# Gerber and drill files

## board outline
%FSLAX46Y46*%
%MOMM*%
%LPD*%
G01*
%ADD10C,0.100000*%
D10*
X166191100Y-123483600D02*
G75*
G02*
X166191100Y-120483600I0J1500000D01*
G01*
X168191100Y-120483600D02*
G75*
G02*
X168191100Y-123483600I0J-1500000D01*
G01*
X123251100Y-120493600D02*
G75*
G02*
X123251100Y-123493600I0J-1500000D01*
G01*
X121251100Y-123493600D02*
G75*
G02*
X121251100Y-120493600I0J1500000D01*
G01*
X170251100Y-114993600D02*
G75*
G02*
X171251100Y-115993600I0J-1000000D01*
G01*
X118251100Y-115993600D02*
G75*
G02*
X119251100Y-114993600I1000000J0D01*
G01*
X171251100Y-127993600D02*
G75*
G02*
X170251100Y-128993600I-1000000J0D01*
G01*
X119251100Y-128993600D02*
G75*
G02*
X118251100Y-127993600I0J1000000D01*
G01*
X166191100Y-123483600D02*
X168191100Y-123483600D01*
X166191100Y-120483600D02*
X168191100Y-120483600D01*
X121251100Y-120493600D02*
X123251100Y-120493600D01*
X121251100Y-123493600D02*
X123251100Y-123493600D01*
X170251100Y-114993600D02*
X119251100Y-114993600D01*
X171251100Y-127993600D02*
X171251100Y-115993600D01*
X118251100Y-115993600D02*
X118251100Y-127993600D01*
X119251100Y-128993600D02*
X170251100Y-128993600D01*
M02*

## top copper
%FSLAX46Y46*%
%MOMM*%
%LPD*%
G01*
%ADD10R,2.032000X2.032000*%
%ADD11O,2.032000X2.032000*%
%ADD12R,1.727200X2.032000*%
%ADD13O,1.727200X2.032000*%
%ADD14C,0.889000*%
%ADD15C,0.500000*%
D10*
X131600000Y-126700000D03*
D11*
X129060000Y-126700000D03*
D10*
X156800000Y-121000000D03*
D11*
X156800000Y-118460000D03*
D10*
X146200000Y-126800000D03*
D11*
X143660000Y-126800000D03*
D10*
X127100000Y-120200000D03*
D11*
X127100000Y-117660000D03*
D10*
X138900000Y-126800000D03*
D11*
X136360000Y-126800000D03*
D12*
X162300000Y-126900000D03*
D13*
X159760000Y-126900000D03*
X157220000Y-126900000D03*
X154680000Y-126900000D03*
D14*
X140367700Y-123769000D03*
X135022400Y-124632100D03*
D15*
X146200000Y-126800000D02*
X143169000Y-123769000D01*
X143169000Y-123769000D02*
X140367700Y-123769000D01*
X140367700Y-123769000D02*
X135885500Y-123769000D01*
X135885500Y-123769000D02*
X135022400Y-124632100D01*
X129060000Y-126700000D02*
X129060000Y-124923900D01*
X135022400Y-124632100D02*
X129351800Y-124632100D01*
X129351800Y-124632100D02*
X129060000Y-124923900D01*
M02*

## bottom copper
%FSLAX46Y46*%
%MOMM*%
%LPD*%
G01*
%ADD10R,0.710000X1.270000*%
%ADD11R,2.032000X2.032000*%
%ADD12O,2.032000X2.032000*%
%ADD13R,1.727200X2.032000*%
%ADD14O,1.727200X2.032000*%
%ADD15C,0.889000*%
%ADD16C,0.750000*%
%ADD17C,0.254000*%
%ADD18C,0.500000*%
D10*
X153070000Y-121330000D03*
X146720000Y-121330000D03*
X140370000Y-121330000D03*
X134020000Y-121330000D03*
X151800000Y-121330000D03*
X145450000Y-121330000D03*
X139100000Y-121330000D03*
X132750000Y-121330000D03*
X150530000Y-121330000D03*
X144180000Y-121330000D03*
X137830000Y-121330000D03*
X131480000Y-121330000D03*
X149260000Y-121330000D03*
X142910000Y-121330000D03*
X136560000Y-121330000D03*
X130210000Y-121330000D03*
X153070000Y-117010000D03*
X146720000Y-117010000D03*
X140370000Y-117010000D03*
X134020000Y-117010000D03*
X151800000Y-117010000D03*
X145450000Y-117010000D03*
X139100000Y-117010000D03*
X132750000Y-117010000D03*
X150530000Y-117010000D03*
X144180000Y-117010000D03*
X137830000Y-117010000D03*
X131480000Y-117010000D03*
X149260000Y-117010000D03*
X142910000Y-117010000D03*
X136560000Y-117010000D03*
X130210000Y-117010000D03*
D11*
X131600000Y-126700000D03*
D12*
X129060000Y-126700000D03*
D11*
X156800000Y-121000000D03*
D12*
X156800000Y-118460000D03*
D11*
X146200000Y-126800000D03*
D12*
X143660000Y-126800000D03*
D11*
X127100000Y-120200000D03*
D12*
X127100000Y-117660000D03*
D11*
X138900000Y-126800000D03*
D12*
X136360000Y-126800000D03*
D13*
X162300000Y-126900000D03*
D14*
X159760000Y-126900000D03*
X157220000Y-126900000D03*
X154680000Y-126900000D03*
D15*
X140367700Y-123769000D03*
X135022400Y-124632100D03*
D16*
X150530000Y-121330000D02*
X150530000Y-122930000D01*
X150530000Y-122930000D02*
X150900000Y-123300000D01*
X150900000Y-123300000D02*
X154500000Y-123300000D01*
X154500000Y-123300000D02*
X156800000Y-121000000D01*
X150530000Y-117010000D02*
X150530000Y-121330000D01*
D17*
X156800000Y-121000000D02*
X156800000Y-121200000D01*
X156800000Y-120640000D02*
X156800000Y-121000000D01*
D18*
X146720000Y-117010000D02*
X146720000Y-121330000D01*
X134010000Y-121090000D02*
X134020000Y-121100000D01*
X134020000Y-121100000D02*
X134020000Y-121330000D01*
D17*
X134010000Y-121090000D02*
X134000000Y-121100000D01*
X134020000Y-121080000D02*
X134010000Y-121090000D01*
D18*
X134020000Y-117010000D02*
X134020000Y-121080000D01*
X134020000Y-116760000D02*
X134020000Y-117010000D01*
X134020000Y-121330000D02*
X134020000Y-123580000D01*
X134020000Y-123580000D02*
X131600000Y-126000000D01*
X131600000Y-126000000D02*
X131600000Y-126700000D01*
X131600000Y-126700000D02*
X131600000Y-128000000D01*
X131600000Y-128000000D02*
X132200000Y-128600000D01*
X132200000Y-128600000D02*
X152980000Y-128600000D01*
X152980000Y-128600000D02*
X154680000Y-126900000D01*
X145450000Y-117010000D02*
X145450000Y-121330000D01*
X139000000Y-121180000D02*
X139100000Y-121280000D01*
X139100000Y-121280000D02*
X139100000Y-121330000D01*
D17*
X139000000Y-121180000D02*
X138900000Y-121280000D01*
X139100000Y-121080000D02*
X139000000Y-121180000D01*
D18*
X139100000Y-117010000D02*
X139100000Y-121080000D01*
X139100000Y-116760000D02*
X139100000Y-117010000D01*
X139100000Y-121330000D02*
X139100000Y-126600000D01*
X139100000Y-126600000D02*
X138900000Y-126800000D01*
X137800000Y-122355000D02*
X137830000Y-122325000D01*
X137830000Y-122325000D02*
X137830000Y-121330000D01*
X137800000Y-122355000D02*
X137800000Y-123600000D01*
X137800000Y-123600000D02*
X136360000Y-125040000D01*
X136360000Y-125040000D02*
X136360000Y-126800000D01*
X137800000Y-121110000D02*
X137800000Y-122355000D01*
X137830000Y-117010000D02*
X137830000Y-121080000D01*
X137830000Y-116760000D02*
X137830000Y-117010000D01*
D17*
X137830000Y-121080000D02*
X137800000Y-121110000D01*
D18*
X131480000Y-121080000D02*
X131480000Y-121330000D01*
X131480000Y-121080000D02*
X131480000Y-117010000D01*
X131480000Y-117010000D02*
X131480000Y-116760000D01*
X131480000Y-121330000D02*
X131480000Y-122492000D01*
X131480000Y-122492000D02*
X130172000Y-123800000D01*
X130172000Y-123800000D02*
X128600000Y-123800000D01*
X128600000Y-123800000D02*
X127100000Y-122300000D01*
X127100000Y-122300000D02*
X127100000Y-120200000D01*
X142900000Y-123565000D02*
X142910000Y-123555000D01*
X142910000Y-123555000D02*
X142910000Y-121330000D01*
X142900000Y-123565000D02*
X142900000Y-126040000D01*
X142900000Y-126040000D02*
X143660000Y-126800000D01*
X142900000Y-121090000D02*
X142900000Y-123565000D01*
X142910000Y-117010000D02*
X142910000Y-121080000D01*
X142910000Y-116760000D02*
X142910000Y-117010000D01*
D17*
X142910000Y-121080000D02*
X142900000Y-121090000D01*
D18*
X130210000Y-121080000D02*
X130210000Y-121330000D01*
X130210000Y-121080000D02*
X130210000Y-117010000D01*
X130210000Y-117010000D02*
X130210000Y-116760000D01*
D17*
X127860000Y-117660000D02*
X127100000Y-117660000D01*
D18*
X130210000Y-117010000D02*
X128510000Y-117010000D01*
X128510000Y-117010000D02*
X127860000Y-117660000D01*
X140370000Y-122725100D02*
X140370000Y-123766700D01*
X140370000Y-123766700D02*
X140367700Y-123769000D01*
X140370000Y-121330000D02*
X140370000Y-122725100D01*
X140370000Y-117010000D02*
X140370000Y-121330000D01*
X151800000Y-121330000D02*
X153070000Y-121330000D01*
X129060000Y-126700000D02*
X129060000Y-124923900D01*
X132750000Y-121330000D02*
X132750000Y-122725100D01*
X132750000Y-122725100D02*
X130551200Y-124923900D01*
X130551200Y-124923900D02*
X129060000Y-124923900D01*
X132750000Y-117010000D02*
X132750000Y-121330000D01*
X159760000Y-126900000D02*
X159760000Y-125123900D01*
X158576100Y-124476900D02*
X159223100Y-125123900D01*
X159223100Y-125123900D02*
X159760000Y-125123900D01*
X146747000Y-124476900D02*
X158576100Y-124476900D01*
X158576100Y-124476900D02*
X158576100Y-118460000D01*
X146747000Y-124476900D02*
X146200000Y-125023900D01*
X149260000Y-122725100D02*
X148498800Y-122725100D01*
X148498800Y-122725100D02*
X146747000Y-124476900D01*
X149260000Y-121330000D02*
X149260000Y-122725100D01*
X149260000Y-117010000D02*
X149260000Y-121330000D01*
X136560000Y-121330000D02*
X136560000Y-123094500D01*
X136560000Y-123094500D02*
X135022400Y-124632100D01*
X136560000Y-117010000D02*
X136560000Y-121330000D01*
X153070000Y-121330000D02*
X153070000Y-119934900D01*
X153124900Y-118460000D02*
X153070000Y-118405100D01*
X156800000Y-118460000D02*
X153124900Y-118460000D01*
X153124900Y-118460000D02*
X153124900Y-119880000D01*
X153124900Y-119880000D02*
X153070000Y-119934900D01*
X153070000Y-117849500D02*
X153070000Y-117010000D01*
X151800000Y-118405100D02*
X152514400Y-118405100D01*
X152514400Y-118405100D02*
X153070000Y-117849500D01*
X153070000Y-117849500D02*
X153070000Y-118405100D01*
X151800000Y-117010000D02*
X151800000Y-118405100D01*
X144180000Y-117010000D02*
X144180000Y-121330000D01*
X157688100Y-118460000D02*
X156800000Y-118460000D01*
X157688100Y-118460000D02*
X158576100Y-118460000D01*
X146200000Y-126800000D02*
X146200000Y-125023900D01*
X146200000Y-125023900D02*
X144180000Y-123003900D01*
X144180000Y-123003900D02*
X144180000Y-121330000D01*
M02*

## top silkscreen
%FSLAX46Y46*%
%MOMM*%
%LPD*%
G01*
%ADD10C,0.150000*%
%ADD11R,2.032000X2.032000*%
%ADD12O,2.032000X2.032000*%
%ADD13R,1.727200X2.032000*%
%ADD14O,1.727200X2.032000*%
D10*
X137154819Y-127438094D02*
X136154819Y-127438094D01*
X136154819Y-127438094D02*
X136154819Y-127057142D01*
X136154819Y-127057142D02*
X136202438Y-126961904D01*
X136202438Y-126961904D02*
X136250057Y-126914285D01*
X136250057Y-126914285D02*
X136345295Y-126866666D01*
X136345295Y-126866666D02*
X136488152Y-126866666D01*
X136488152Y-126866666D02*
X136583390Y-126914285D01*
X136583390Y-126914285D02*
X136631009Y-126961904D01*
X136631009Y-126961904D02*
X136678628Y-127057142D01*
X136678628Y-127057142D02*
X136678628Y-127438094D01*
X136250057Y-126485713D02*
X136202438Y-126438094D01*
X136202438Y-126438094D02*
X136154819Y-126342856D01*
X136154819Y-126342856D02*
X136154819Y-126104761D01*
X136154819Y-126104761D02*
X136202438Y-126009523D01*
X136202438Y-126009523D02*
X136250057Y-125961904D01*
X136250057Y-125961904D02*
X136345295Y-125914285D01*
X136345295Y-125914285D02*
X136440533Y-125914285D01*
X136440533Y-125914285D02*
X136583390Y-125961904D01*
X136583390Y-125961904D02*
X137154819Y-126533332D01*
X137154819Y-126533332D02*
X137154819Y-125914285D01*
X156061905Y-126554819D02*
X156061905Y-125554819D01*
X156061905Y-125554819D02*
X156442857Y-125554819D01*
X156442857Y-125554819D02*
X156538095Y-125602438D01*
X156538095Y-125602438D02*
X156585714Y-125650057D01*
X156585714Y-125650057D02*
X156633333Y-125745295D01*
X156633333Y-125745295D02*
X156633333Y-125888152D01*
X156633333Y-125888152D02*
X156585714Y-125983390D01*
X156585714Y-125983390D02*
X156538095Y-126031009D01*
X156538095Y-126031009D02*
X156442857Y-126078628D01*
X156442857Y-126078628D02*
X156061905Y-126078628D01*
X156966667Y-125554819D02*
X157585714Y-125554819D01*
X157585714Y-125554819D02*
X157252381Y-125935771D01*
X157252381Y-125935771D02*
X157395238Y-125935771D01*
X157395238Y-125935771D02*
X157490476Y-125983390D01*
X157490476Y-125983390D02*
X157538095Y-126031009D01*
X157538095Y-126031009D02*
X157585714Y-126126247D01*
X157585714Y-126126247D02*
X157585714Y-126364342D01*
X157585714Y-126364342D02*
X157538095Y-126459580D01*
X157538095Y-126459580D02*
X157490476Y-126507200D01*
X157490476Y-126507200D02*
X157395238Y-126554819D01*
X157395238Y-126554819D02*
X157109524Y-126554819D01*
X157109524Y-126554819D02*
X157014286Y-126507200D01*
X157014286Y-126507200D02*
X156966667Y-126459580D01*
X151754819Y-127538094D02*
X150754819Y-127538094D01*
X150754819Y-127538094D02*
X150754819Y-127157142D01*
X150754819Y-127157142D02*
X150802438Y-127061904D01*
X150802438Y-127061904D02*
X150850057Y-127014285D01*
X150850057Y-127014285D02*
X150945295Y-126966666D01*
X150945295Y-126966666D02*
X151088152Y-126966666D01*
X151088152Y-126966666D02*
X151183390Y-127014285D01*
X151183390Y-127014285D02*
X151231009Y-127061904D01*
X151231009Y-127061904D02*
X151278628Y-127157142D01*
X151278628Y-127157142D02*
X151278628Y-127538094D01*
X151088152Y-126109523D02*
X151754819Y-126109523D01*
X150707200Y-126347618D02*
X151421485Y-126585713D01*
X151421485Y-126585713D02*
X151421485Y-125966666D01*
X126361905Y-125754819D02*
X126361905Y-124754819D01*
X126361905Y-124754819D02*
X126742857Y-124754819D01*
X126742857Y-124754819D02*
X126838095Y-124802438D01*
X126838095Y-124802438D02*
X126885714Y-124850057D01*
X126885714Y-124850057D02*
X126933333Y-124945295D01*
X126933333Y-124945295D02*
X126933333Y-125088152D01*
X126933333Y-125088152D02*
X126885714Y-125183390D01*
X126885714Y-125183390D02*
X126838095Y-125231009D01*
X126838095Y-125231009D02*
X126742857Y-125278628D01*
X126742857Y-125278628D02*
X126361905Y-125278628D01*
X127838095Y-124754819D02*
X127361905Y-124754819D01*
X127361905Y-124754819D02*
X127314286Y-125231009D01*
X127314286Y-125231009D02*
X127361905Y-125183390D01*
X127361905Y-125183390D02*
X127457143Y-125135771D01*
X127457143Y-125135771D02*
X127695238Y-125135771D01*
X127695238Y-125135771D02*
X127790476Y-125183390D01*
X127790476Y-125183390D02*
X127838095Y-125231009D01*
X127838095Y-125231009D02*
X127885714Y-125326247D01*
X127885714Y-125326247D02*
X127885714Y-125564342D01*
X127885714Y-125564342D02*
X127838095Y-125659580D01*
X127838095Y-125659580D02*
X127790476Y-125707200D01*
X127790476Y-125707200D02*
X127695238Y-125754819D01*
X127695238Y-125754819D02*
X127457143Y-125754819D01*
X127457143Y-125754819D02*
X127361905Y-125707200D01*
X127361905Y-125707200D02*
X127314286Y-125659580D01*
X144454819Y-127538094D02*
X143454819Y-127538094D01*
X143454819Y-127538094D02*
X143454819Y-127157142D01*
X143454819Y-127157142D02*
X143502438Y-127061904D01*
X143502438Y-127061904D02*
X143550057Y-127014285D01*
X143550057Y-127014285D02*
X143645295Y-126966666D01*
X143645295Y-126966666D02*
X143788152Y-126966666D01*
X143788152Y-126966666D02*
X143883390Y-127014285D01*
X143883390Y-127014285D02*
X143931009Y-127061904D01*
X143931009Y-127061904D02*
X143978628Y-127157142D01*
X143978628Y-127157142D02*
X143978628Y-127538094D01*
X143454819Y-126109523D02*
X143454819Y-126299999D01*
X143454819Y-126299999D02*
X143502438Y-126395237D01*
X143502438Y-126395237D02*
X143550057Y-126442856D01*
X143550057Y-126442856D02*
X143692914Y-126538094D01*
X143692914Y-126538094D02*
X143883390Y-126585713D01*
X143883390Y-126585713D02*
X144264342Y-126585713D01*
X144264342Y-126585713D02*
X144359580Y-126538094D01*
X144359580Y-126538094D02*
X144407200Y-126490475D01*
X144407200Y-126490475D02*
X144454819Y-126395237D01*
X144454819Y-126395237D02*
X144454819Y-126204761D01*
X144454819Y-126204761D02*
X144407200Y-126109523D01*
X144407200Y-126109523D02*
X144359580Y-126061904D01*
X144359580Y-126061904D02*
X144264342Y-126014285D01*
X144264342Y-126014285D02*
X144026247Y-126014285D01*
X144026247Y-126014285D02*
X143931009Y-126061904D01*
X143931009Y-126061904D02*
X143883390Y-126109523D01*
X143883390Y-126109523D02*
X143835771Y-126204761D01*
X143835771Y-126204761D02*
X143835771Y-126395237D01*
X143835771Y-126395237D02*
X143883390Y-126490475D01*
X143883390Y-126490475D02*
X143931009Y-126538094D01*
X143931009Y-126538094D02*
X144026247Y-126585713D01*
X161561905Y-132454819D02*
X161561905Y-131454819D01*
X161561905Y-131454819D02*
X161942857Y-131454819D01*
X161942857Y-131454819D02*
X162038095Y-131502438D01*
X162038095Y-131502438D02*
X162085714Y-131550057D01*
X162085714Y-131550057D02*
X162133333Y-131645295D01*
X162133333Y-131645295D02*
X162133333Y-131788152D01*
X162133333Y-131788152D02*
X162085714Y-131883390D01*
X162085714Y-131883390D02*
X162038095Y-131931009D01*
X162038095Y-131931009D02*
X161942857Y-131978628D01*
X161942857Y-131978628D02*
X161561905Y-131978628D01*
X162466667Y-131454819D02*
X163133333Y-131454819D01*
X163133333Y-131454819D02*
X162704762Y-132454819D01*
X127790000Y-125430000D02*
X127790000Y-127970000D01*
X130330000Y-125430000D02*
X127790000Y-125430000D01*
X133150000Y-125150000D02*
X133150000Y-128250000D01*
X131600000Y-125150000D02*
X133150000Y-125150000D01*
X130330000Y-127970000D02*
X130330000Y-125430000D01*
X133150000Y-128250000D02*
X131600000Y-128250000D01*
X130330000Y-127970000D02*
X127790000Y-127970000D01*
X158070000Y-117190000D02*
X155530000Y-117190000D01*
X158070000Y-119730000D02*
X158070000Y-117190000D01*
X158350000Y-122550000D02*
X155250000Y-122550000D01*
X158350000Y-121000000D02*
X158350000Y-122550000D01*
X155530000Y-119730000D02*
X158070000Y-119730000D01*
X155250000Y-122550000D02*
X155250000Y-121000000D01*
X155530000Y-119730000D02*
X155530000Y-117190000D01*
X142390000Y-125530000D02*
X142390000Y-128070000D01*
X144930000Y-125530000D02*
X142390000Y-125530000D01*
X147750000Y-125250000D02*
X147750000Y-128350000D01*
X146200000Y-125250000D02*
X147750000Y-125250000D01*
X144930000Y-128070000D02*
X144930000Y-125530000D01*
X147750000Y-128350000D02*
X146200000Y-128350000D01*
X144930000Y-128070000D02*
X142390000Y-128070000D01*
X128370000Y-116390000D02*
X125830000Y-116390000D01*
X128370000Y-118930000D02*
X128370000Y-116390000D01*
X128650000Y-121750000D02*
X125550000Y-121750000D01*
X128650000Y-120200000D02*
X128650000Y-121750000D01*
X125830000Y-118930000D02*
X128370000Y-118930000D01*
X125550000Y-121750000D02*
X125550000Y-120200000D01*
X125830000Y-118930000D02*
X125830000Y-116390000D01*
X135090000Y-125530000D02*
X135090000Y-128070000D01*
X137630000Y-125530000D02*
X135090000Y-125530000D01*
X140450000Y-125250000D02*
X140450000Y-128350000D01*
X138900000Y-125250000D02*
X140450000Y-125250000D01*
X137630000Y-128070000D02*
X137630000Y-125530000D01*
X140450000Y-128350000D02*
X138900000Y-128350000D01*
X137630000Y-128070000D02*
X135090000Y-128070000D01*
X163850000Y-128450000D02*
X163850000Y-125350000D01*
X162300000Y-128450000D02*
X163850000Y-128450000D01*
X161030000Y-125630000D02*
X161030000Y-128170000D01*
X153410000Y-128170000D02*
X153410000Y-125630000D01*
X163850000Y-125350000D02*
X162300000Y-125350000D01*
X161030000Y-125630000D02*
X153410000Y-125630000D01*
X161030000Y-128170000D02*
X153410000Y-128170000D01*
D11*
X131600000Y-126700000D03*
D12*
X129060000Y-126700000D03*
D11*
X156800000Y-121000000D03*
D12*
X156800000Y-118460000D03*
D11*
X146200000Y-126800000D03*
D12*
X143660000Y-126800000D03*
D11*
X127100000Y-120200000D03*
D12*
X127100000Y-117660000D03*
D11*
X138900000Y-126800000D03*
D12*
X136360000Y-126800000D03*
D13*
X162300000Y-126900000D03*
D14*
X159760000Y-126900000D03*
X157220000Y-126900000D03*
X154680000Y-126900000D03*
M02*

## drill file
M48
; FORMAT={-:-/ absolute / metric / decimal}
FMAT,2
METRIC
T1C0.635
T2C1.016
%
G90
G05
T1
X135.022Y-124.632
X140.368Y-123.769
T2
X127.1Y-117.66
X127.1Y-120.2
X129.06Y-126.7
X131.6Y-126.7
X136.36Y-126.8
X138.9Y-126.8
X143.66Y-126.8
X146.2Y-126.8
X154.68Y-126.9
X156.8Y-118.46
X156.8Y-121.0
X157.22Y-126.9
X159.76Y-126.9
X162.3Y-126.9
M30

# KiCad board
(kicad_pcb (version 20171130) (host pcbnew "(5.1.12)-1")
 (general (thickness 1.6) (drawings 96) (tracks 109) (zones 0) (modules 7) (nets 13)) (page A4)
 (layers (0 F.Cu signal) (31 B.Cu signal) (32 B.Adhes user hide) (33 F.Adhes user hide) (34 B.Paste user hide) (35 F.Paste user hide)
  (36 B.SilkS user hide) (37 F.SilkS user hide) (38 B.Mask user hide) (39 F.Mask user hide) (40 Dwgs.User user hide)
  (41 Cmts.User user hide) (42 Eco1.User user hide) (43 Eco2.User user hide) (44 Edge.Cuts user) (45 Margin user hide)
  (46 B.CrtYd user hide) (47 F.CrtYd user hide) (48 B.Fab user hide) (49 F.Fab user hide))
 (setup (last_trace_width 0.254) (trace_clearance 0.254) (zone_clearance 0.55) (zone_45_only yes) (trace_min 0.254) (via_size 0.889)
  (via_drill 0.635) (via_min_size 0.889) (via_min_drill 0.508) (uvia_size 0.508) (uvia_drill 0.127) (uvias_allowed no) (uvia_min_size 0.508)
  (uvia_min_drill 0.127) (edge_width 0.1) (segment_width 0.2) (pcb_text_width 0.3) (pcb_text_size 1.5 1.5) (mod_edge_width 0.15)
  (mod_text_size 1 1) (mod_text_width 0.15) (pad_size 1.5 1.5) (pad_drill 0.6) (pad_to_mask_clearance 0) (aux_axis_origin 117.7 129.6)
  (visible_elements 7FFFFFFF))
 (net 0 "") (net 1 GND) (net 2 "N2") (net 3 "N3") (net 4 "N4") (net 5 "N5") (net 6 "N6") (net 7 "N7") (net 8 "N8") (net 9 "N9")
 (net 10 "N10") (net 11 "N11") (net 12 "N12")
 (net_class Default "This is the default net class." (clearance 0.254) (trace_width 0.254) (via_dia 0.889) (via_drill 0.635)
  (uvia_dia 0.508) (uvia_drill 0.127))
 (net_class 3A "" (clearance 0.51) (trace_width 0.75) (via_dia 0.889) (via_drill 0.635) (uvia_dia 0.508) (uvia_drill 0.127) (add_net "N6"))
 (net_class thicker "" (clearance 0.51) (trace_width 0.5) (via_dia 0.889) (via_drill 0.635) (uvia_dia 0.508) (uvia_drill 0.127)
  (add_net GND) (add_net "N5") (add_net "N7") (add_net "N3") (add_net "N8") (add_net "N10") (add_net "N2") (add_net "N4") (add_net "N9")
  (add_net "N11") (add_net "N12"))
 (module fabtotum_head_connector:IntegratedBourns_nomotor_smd (layer B.Cu) (at 153 121.35 90)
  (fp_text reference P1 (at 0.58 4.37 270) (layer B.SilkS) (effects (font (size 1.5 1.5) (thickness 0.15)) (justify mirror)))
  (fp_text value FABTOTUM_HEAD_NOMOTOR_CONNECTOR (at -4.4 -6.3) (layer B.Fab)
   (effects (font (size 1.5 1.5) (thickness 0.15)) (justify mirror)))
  (pad 1 smd rect (at 0.02 0.07 90) (size 1.27 0.71) (layers B.Cu B.Paste B.Mask) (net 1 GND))
  (pad 5 smd rect (at 0.02 -6.28 90) (size 1.27 0.71) (layers B.Cu B.Paste B.Mask) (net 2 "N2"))
  (pad 9 smd rect (at 0.02 -12.63 90) (size 1.27 0.71) (layers B.Cu B.Paste B.Mask) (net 1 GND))
  (pad 13 smd rect (at 0.02 -18.98 90) (size 1.27 0.71) (layers B.Cu B.Paste B.Mask) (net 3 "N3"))
  (pad 2 smd rect (at 0.02 -1.2 90) (size 1.27 0.71) (layers B.Cu B.Paste B.Mask) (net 1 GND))
  (pad 6 smd rect (at 0.02 -7.55 90) (size 1.27 0.71) (layers B.Cu B.Paste B.Mask) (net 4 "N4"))
  (pad 10 smd rect (at 0.02 -13.9 90) (size 1.27 0.71) (layers B.Cu B.Paste B.Mask) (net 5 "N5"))
  (pad 14 smd rect (at 0.02 -20.25 90) (size 1.27 0.71) (layers B.Cu B.Paste B.Mask) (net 1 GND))
  (pad 3 smd rect (at 0.02 -2.47 90) (size 1.27 0.71) (layers B.Cu B.Paste B.Mask) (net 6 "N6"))
  (pad 7 smd rect (at 0.02 -8.82 90) (size 1.27 0.71) (layers B.Cu B.Paste B.Mask) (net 1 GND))
  (pad 11 smd rect (at 0.02 -15.17 90) (size 1.27 0.71) (layers B.Cu B.Paste B.Mask) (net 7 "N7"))
  (pad 15 smd rect (at 0.02 -21.52 90) (size 1.27 0.71) (layers B.Cu B.Paste B.Mask) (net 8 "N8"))
  (pad 4 smd rect (at 0.02 -3.74 90) (size 1.27 0.71) (layers B.Cu B.Paste B.Mask) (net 1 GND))
  (pad 8 smd rect (at 0.02 -10.09 90) (size 1.27 0.71) (layers B.Cu B.Paste B.Mask) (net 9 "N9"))
  (pad 12 smd rect (at 0.02 -16.44 90) (size 1.27 0.71) (layers B.Cu B.Paste B.Mask) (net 1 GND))
  (pad 16 smd rect (at 0.02 -22.79 90) (size 1.27 0.71) (layers B.Cu B.Paste B.Mask) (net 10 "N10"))
  (pad 1 smd rect (at 4.34 0.07 90) (size 1.27 0.71) (layers B.Cu B.Paste B.Mask) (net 1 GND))
  (pad 5 smd rect (at 4.34 -6.28 90) (size 1.27 0.71) (layers B.Cu B.Paste B.Mask) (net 2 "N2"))
  (pad 9 smd rect (at 4.34 -12.63 90) (size 1.27 0.71) (layers B.Cu B.Paste B.Mask) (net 1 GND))
  (pad 13 smd rect (at 4.34 -18.98 90) (size 1.27 0.71) (layers B.Cu B.Paste B.Mask) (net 3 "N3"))
  (pad 2 smd rect (at 4.34 -1.2 90) (size 1.27 0.71) (layers B.Cu B.Paste B.Mask) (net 1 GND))
  (pad 6 smd rect (at 4.34 -7.55 90) (size 1.27 0.71) (layers B.Cu B.Paste B.Mask) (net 4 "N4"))
  (pad 10 smd rect (at 4.34 -13.9 90) (size 1.27 0.71) (layers B.Cu B.Paste B.Mask) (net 5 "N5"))
  (pad 14 smd rect (at 4.34 -20.25 90) (size 1.27 0.71) (layers B.Cu B.Paste B.Mask) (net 1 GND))
  (pad 3 smd rect (at 4.34 -2.47 90) (size 1.27 0.71) (layers B.Cu B.Paste B.Mask) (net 6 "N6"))
  (pad 7 smd rect (at 4.34 -8.82 90) (size 1.27 0.71) (layers B.Cu B.Paste B.Mask) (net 1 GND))
  (pad 11 smd rect (at 4.34 -15.17 90) (size 1.27 0.71) (layers B.Cu B.Paste B.Mask) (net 7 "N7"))
  (pad 15 smd rect (at 4.34 -21.52 90) (size 1.27 0.71) (layers B.Cu B.Paste B.Mask) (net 8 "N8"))
  (pad 4 smd rect (at 4.34 -3.74 90) (size 1.27 0.71) (layers B.Cu B.Paste B.Mask) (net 1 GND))
  (pad 8 smd rect (at 4.34 -10.09 90) (size 1.27 0.71) (layers B.Cu B.Paste B.Mask) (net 9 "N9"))
  (pad 12 smd rect (at 4.34 -16.44 90) (size 1.27 0.71) (layers B.Cu B.Paste B.Mask) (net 1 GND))
  (pad 16 smd rect (at 4.34 -22.79 90) (size 1.27 0.71) (layers B.Cu B.Paste B.Mask) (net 10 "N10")))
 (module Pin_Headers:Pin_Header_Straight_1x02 (layer F.Cu) (at 131.6 126.7 270)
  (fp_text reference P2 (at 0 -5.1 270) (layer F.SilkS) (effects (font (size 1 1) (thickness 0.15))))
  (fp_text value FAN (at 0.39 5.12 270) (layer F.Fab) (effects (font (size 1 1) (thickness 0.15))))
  (fp_line (start -1.27 3.81) (end 1.27 3.81) (layer F.SilkS) (width 0.15))
  (fp_line (start -1.27 1.27) (end -1.27 3.81) (layer F.SilkS) (width 0.15))
  (fp_line (start -1.55 -1.55) (end 1.55 -1.55) (layer F.SilkS) (width 0.15))
  (fp_line (start -1.55 0) (end -1.55 -1.55) (layer F.SilkS) (width 0.15))
  (fp_line (start 1.27 1.27) (end -1.27 1.27) (layer F.SilkS) (width 0.15))
  (fp_line (start 1.55 -1.55) (end 1.55 0) (layer F.SilkS) (width 0.15))
  (fp_line (start 1.27 1.27) (end 1.27 3.81) (layer F.SilkS) (width 0.15))
  (pad 1 thru_hole rect (at 0 0 270) (size 2.032 2.032) (drill 1.016) (layers *.Cu *.Mask F.SilkS) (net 3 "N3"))
  (pad 2 thru_hole oval (at 0 2.54 270) (size 2.032 2.032) (drill 1.016) (layers *.Cu *.Mask F.SilkS) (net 1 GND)))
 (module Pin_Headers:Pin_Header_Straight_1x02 (layer F.Cu) (at 156.8 121 180)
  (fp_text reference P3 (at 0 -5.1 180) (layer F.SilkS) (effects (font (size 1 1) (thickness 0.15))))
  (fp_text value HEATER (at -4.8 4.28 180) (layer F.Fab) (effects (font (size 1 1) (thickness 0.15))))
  (fp_line (start -1.27 3.81) (end 1.27 3.81) (layer F.SilkS) (width 0.15))
  (fp_line (start -1.27 1.27) (end -1.27 3.81) (layer F.SilkS) (width 0.15))
  (fp_line (start -1.55 -1.55) (end 1.55 -1.55) (layer F.SilkS) (width 0.15))
  (fp_line (start -1.55 0) (end -1.55 -1.55) (layer F.SilkS) (width 0.15))
  (fp_line (start 1.27 1.27) (end -1.27 1.27) (layer F.SilkS) (width 0.15))
  (fp_line (start 1.55 -1.55) (end 1.55 0) (layer F.SilkS) (width 0.15))
  (fp_line (start 1.27 1.27) (end 1.27 3.81) (layer F.SilkS) (width 0.15))
  (pad 1 thru_hole rect (at 0 0 180) (size 2.032 2.032) (drill 1.016) (layers *.Cu *.Mask F.SilkS) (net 6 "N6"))
  (pad 2 thru_hole oval (at 0 2.54 180) (size 2.032 2.032) (drill 1.016) (layers *.Cu *.Mask F.SilkS) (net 1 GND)))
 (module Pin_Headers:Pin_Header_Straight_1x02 (layer F.Cu) (at 146.2 126.8 270)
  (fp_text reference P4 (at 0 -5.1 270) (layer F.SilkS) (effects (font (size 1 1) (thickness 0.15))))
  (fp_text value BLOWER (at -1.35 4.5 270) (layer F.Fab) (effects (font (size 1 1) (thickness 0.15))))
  (fp_line (start -1.27 3.81) (end 1.27 3.81) (layer F.SilkS) (width 0.15))
  (fp_line (start -1.27 1.27) (end -1.27 3.81) (layer F.SilkS) (width 0.15))
  (fp_line (start -1.55 -1.55) (end 1.55 -1.55) (layer F.SilkS) (width 0.15))
  (fp_line (start -1.55 0) (end -1.55 -1.55) (layer F.SilkS) (width 0.15))
  (fp_line (start 1.27 1.27) (end -1.27 1.27) (layer F.SilkS) (width 0.15))
  (fp_line (start 1.55 -1.55) (end 1.55 0) (layer F.SilkS) (width 0.15))
  (fp_line (start 1.27 1.27) (end 1.27 3.81) (layer F.SilkS) (width 0.15))
  (pad 1 thru_hole rect (at 0 0 270) (size 2.032 2.032) (drill 1.016) (layers *.Cu *.Mask F.SilkS) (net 1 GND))
  (pad 2 thru_hole oval (at 0 2.54 270) (size 2.032 2.032) (drill 1.016) (layers *.Cu *.Mask F.SilkS) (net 9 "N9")))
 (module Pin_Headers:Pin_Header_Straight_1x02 (layer F.Cu) (at 127.1 120.2 180)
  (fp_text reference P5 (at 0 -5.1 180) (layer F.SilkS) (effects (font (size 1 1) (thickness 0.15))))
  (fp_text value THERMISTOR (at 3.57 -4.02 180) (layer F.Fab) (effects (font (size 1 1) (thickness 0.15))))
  (fp_line (start -1.27 3.81) (end 1.27 3.81) (layer F.SilkS) (width 0.15))
  (fp_line (start -1.27 1.27) (end -1.27 3.81) (layer F.SilkS) (width 0.15))
  (fp_line (start -1.55 -1.55) (end 1.55 -1.55) (layer F.SilkS) (width 0.15))
  (fp_line (start -1.55 0) (end -1.55 -1.55) (layer F.SilkS) (width 0.15))
  (fp_line (start 1.27 1.27) (end -1.27 1.27) (layer F.SilkS) (width 0.15))
  (fp_line (start 1.55 -1.55) (end 1.55 0) (layer F.SilkS) (width 0.15))
  (fp_line (start 1.27 1.27) (end 1.27 3.81) (layer F.SilkS) (width 0.15))
  (pad 1 thru_hole rect (at 0 0 180) (size 2.032 2.032) (drill 1.016) (layers *.Cu *.Mask F.SilkS) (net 8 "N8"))
  (pad 2 thru_hole oval (at 0 2.54 180) (size 2.032 2.032) (drill 1.016) (layers *.Cu *.Mask F.SilkS) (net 10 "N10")))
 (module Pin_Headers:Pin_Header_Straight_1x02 (layer F.Cu) (at 138.9 126.8 270)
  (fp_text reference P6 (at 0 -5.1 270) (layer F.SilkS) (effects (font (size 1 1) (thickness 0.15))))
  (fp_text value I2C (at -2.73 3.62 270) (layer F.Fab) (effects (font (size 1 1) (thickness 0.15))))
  (fp_line (start -1.27 3.81) (end 1.27 3.81) (layer F.SilkS) (width 0.15))
  (fp_line (start -1.27 1.27) (end -1.27 3.81) (layer F.SilkS) (width 0.15))
  (fp_line (start -1.55 -1.55) (end 1.55 -1.55) (layer F.SilkS) (width 0.15))
  (fp_line (start -1.55 0) (end -1.55 -1.55) (layer F.SilkS) (width 0.15))
  (fp_line (start 1.27 1.27) (end -1.27 1.27) (layer F.SilkS) (width 0.15))
  (fp_line (start 1.55 -1.55) (end 1.55 0) (layer F.SilkS) (width 0.15))
  (fp_line (start 1.27 1.27) (end 1.27 3.81) (layer F.SilkS) (width 0.15))
  (pad 1 thru_hole rect (at 0 0 270) (size 2.032 2.032) (drill 1.016) (layers *.Cu *.Mask F.SilkS) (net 5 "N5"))
  (pad 2 thru_hole oval (at 0 2.54 270) (size 2.032 2.032) (drill 1.016) (layers *.Cu *.Mask F.SilkS) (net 7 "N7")))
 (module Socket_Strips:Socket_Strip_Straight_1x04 (layer F.Cu) (at 162.3 126.9 180)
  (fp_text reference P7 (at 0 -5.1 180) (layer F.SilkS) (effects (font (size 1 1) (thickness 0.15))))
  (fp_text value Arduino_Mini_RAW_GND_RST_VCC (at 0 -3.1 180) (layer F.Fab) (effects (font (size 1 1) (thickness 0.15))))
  (fp_line (start -1.55 -1.55) (end -1.55 1.55) (layer F.SilkS) (width 0.15))
  (fp_line (start 0 -1.55) (end -1.55 -1.55) (layer F.SilkS) (width 0.15))
  (fp_line (start 1.27 1.27) (end 1.27 -1.27) (layer F.SilkS) (width 0.15))
  (fp_line (start 8.89 -1.27) (end 8.89 1.27) (layer F.SilkS) (width 0.15))
  (fp_line (start -1.55 1.55) (end 0 1.55) (layer F.SilkS) (width 0.15))
  (fp_line (start 1.27 1.27) (end 8.89 1.27) (layer F.SilkS) (width 0.15))
  (fp_line (start 1.27 -1.27) (end 8.89 -1.27) (layer F.SilkS) (width 0.15))
  (pad 1 thru_hole rect (at 0 0 180) (size 1.7272 2.032) (drill 1.016) (layers *.Cu *.Mask F.SilkS) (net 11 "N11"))
  (pad 2 thru_hole oval (at 2.54 0 180) (size 1.7272 2.032) (drill 1.016) (layers *.Cu *.Mask F.SilkS) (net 1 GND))
  (pad 3 thru_hole oval (at 5.08 0 180) (size 1.7272 2.032) (drill 1.016) (layers *.Cu *.Mask F.SilkS) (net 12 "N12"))
  (pad 4 thru_hole oval (at 7.62 0 180) (size 1.7272 2.032) (drill 1.016) (layers *.Cu *.Mask F.SilkS) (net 3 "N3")))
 (gr_arc (start 166.1911 121.9836) (end 166.1911 120.4836) (angle -180) (layer Edge.Cuts) (width 0.1))
 (gr_arc (start 168.1911 121.9836) (end 168.1911 123.4836) (angle -180) (layer Edge.Cuts) (width 0.1))
 (gr_arc (start 123.2511 121.9936) (end 123.2511 123.4936) (angle -180) (layer Edge.Cuts) (width 0.1))
 (gr_arc (start 121.2511 121.9936) (end 121.2511 120.4936) (angle -180) (layer Edge.Cuts) (width 0.1))
 (gr_arc (start 170.2511 115.9936) (end 171.2511 115.9936) (angle -90) (layer Edge.Cuts) (width 0.1))
 (gr_arc (start 119.2511 115.9936) (end 119.2511 114.9936) (angle -90) (layer Edge.Cuts) (width 0.1))
 (gr_arc (start 170.2511 127.9936) (end 170.2511 128.9936) (angle -90) (layer Edge.Cuts) (width 0.1))
 (gr_arc (start 119.2511 127.9936) (end 118.2511 127.9936) (angle -90) (layer Edge.Cuts) (width 0.1))
 (gr_line (start 166.1911 123.4836) (end 168.1911 123.4836) (layer Edge.Cuts) (width 0.1))
 (gr_line (start 166.1911 120.4836) (end 168.1911 120.4836) (layer Edge.Cuts) (width 0.1))
 (gr_line (start 121.2511 120.4936) (end 123.2511 120.4936) (layer Edge.Cuts) (width 0.1))
 (gr_line (start 121.2511 123.4936) (end 123.2511 123.4936) (layer Edge.Cuts) (width 0.1))
 (gr_line (start 170.2511 114.9936) (end 119.2511 114.9936) (layer Edge.Cuts) (width 0.1))
 (gr_line (start 171.2511 127.9936) (end 171.2511 115.9936) (layer Edge.Cuts) (width 0.1))
 (gr_line (start 118.2511 115.9936) (end 118.2511 127.9936) (layer Edge.Cuts) (width 0.1))
 (gr_line (start 119.2511 128.9936) (end 170.2511 128.9936) (layer Edge.Cuts) (width 0.1))
 (segment (start 150.53 121.33) (end 150.53 122.93) (width 0.75) (layer B.Cu) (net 6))
 (segment (start 150.53 122.93) (end 150.9 123.3) (width 0.75) (layer B.Cu) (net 6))
 (segment (start 150.9 123.3) (end 154.5 123.3) (width 0.75) (layer B.Cu) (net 6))
 (segment (start 154.5 123.3) (end 156.8 121) (width 0.75) (layer B.Cu) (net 6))
 (segment (start 150.53 117.01) (end 150.53 121.33) (width 0.75) (layer B.Cu) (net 6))
 (segment (start 156.8 121) (end 156.8 121.2) (width 0.254) (layer B.Cu) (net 6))
 (segment (start 156.8 120.64) (end 156.8 121) (width 0.254) (layer B.Cu) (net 6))
 (segment (start 146.72 117.01) (end 146.72 121.33) (width 0.5) (layer B.Cu) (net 2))
 (segment (start 134.01 121.09) (end 134.02 121.1) (width 0.5) (layer B.Cu) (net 3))
 (segment (start 134.02 121.1) (end 134.02 121.33) (width 0.5) (layer B.Cu) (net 3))
 (segment (start 134.01 121.09) (end 134 121.1) (width 0.254) (layer B.Cu) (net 3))
 (segment (start 134.02 121.08) (end 134.01 121.09) (width 0.254) (layer B.Cu) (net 3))
 (segment (start 134.02 117.01) (end 134.02 121.08) (width 0.5) (layer B.Cu) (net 3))
 (segment (start 134.02 116.76) (end 134.02 117.01) (width 0.5) (layer B.Cu) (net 3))
 (segment (start 134.02 121.33) (end 134.02 123.58) (width 0.5) (layer B.Cu) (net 3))
 (segment (start 134.02 123.58) (end 131.6 126) (width 0.5) (layer B.Cu) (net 3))
 (segment (start 131.6 126) (end 131.6 126.7) (width 0.5) (layer B.Cu) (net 3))
 (segment (start 131.6 126.7) (end 131.6 128) (width 0.5) (layer B.Cu) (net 3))
 (segment (start 131.6 128) (end 132.2 128.6) (width 0.5) (layer B.Cu) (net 3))
 (segment (start 132.2 128.6) (end 152.98 128.6) (width 0.5) (layer B.Cu) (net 3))
 (segment (start 152.98 128.6) (end 154.68 126.9) (width 0.5) (layer B.Cu) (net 3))
 (segment (start 145.45 117.01) (end 145.45 121.33) (width 0.5) (layer B.Cu) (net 4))
 (segment (start 139 121.18) (end 139.1 121.28) (width 0.5) (layer B.Cu) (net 5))
 (segment (start 139.1 121.28) (end 139.1 121.33) (width 0.5) (layer B.Cu) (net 5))
 (segment (start 139 121.18) (end 138.9 121.28) (width 0.254) (layer B.Cu) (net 5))
 (segment (start 139.1 121.08) (end 139 121.18) (width 0.254) (layer B.Cu) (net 5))
 (segment (start 139.1 117.01) (end 139.1 121.08) (width 0.5) (layer B.Cu) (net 5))
 (segment (start 139.1 116.76) (end 139.1 117.01) (width 0.5) (layer B.Cu) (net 5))
 (segment (start 139.1 121.33) (end 139.1 126.6) (width 0.5) (layer B.Cu) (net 5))
 (segment (start 139.1 126.6) (end 138.9 126.8) (width 0.5) (layer B.Cu) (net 5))
 (segment (start 137.8 122.355) (end 137.83 122.325) (width 0.5) (layer B.Cu) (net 7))
 (segment (start 137.83 122.325) (end 137.83 121.33) (width 0.5) (layer B.Cu) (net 7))
 (segment (start 137.8 122.355) (end 137.8 123.6) (width 0.5) (layer B.Cu) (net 7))
 (segment (start 137.8 123.6) (end 136.36 125.04) (width 0.5) (layer B.Cu) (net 7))
 (segment (start 136.36 125.04) (end 136.36 126.8) (width 0.5) (layer B.Cu) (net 7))
 (segment (start 137.8 121.11) (end 137.8 122.355) (width 0.5) (layer B.Cu) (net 7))
 (segment (start 137.83 117.01) (end 137.83 121.08) (width 0.5) (layer B.Cu) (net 7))
 (segment (start 137.83 116.76) (end 137.83 117.01) (width 0.5) (layer B.Cu) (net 7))
 (segment (start 137.83 121.08) (end 137.8 121.11) (width 0.254) (layer B.Cu) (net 7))
 (segment (start 131.48 121.08) (end 131.48 121.33) (width 0.5) (layer B.Cu) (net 8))
 (segment (start 131.48 121.08) (end 131.48 117.01) (width 0.5) (layer B.Cu) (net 8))
 (segment (start 131.48 117.01) (end 131.48 116.76) (width 0.5) (layer B.Cu) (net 8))
 (segment (start 131.48 121.33) (end 131.48 122.492) (width 0.5) (layer B.Cu) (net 8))
 (segment (start 131.48 122.492) (end 130.172 123.8) (width 0.5) (layer B.Cu) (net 8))
 (segment (start 130.172 123.8) (end 128.6 123.8) (width 0.5) (layer B.Cu) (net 8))
 (segment (start 128.6 123.8) (end 127.1 122.3) (width 0.5) (layer B.Cu) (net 8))
 (segment (start 127.1 122.3) (end 127.1 120.2) (width 0.5) (layer B.Cu) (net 8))
 (segment (start 142.9 123.565) (end 142.91 123.555) (width 0.5) (layer B.Cu) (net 9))
 (segment (start 142.91 123.555) (end 142.91 121.33) (width 0.5) (layer B.Cu) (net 9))
 (segment (start 142.9 123.565) (end 142.9 126.04) (width 0.5) (layer B.Cu) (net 9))
 (segment (start 142.9 126.04) (end 143.66 126.8) (width 0.5) (layer B.Cu) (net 9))
 (segment (start 142.9 121.09) (end 142.9 123.565) (width 0.5) (layer B.Cu) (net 9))
 (segment (start 142.91 117.01) (end 142.91 121.08) (width 0.5) (layer B.Cu) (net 9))
 (segment (start 142.91 116.76) (end 142.91 117.01) (width 0.5) (layer B.Cu) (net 9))
 (segment (start 142.91 121.08) (end 142.9 121.09) (width 0.254) (layer B.Cu) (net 9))
 (segment (start 130.21 121.08) (end 130.21 121.33) (width 0.5) (layer B.Cu) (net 10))
 (segment (start 130.21 121.08) (end 130.21 117.01) (width 0.5) (layer B.Cu) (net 10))
 (segment (start 130.21 117.01) (end 130.21 116.76) (width 0.5) (layer B.Cu) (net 10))
 (segment (start 127.86 117.66) (end 127.1 117.66) (width 0.254) (layer B.Cu) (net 10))
 (segment (start 130.21 117.01) (end 128.51 117.01) (width 0.5) (layer B.Cu) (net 10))
 (segment (start 128.51 117.01) (end 127.86 117.66) (width 0.5) (layer B.Cu) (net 10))
 (segment (start 146.2 126.8) (end 143.169 123.769) (width 0.5) (layer F.Cu) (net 1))
 (segment (start 143.169 123.769) (end 140.3677 123.769) (width 0.5) (layer F.Cu) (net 1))
 (segment (start 140.3677 123.769) (end 135.8855 123.769) (width 0.5) (layer F.Cu) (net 1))
 (segment (start 135.8855 123.769) (end 135.0224 124.6321) (width 0.5) (layer F.Cu) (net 1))
 (segment (start 140.37 122.7251) (end 140.37 123.7667) (width 0.5) (layer B.Cu) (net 1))
 (segment (start 140.37 123.7667) (end 140.3677 123.769) (width 0.5) (layer B.Cu) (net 1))
 (segment (start 140.37 121.33) (end 140.37 122.7251) (width 0.5) (layer B.Cu) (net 1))
 (segment (start 140.37 117.01) (end 140.37 121.33) (width 0.5) (layer B.Cu) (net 1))
 (segment (start 151.8 121.33) (end 153.07 121.33) (width 0.5) (layer B.Cu) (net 1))
 (segment (start 129.06 126.7) (end 129.06 124.9239) (width 0.5) (layer B.Cu) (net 1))
 (segment (start 132.75 121.33) (end 132.75 122.7251) (width 0.5) (layer B.Cu) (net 1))
 (segment (start 132.75 122.7251) (end 130.5512 124.9239) (width 0.5) (layer B.Cu) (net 1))
 (segment (start 130.5512 124.9239) (end 129.06 124.9239) (width 0.5) (layer B.Cu) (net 1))
 (segment (start 132.75 117.01) (end 132.75 121.33) (width 0.5) (layer B.Cu) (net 1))
 (segment (start 159.76 126.9) (end 159.76 125.1239) (width 0.5) (layer B.Cu) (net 1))
 (segment (start 158.5761 124.4769) (end 159.2231 125.1239) (width 0.5) (layer B.Cu) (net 1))
 (segment (start 159.2231 125.1239) (end 159.76 125.1239) (width 0.5) (layer B.Cu) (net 1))
 (segment (start 146.747 124.4769) (end 158.5761 124.4769) (width 0.5) (layer B.Cu) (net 1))
 (segment (start 158.5761 124.4769) (end 158.5761 118.46) (width 0.5) (layer B.Cu) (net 1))
 (segment (start 146.747 124.4769) (end 146.2 125.0239) (width 0.5) (layer B.Cu) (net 1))
 (segment (start 149.26 122.7251) (end 148.4988 122.7251) (width 0.5) (layer B.Cu) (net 1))
 (segment (start 148.4988 122.7251) (end 146.747 124.4769) (width 0.5) (layer B.Cu) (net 1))
 (segment (start 149.26 121.33) (end 149.26 122.7251) (width 0.5) (layer B.Cu) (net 1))
 (segment (start 149.26 117.01) (end 149.26 121.33) (width 0.5) (layer B.Cu) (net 1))
 (segment (start 129.06 126.7) (end 129.06 124.9239) (width 0.5) (layer F.Cu) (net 1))
 (segment (start 135.0224 124.6321) (end 129.3518 124.6321) (width 0.5) (layer F.Cu) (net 1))
 (segment (start 129.3518 124.6321) (end 129.06 124.9239) (width 0.5) (layer F.Cu) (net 1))
 (segment (start 136.56 121.33) (end 136.56 123.0945) (width 0.5) (layer B.Cu) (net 1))
 (segment (start 136.56 123.0945) (end 135.0224 124.6321) (width 0.5) (layer B.Cu) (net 1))
 (segment (start 136.56 117.01) (end 136.56 121.33) (width 0.5) (layer B.Cu) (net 1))
 (segment (start 153.07 121.33) (end 153.07 119.9349) (width 0.5) (layer B.Cu) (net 1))
 (segment (start 153.1249 118.46) (end 153.07 118.4051) (width 0.5) (layer B.Cu) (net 1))
 (segment (start 156.8 118.46) (end 153.1249 118.46) (width 0.5) (layer B.Cu) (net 1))
 (segment (start 153.1249 118.46) (end 153.1249 119.88) (width 0.5) (layer B.Cu) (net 1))
 (segment (start 153.1249 119.88) (end 153.07 119.9349) (width 0.5) (layer B.Cu) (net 1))
 (segment (start 153.07 117.8495) (end 153.07 117.01) (width 0.5) (layer B.Cu) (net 1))
 (segment (start 151.8 118.4051) (end 152.5144 118.4051) (width 0.5) (layer B.Cu) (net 1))
 (segment (start 152.5144 118.4051) (end 153.07 117.8495) (width 0.5) (layer B.Cu) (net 1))
 (segment (start 153.07 117.8495) (end 153.07 118.4051) (width 0.5) (layer B.Cu) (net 1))
 (segment (start 151.8 117.01) (end 151.8 118.4051) (width 0.5) (layer B.Cu) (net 1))
 (segment (start 144.18 117.01) (end 144.18 121.33) (width 0.5) (layer B.Cu) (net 1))
 (segment (start 157.6881 118.46) (end 156.8 118.46) (width 0.5) (layer B.Cu) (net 1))
 (segment (start 157.6881 118.46) (end 158.5761 118.46) (width 0.5) (layer B.Cu) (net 1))
 (segment (start 146.2 126.8) (end 146.2 125.0239) (width 0.5) (layer B.Cu) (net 1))
 (segment (start 146.2 125.0239) (end 144.18 123.0039) (width 0.5) (layer B.Cu) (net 1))
 (segment (start 144.18 123.0039) (end 144.18 121.33) (width 0.5) (layer B.Cu) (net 1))
 (via (at 140.3677 123.769) (size 0.889) (layers F.Cu B.Cu) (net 1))
 (via (at 135.0224 124.6321) (size 0.889) (layers F.Cu B.Cu) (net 1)))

